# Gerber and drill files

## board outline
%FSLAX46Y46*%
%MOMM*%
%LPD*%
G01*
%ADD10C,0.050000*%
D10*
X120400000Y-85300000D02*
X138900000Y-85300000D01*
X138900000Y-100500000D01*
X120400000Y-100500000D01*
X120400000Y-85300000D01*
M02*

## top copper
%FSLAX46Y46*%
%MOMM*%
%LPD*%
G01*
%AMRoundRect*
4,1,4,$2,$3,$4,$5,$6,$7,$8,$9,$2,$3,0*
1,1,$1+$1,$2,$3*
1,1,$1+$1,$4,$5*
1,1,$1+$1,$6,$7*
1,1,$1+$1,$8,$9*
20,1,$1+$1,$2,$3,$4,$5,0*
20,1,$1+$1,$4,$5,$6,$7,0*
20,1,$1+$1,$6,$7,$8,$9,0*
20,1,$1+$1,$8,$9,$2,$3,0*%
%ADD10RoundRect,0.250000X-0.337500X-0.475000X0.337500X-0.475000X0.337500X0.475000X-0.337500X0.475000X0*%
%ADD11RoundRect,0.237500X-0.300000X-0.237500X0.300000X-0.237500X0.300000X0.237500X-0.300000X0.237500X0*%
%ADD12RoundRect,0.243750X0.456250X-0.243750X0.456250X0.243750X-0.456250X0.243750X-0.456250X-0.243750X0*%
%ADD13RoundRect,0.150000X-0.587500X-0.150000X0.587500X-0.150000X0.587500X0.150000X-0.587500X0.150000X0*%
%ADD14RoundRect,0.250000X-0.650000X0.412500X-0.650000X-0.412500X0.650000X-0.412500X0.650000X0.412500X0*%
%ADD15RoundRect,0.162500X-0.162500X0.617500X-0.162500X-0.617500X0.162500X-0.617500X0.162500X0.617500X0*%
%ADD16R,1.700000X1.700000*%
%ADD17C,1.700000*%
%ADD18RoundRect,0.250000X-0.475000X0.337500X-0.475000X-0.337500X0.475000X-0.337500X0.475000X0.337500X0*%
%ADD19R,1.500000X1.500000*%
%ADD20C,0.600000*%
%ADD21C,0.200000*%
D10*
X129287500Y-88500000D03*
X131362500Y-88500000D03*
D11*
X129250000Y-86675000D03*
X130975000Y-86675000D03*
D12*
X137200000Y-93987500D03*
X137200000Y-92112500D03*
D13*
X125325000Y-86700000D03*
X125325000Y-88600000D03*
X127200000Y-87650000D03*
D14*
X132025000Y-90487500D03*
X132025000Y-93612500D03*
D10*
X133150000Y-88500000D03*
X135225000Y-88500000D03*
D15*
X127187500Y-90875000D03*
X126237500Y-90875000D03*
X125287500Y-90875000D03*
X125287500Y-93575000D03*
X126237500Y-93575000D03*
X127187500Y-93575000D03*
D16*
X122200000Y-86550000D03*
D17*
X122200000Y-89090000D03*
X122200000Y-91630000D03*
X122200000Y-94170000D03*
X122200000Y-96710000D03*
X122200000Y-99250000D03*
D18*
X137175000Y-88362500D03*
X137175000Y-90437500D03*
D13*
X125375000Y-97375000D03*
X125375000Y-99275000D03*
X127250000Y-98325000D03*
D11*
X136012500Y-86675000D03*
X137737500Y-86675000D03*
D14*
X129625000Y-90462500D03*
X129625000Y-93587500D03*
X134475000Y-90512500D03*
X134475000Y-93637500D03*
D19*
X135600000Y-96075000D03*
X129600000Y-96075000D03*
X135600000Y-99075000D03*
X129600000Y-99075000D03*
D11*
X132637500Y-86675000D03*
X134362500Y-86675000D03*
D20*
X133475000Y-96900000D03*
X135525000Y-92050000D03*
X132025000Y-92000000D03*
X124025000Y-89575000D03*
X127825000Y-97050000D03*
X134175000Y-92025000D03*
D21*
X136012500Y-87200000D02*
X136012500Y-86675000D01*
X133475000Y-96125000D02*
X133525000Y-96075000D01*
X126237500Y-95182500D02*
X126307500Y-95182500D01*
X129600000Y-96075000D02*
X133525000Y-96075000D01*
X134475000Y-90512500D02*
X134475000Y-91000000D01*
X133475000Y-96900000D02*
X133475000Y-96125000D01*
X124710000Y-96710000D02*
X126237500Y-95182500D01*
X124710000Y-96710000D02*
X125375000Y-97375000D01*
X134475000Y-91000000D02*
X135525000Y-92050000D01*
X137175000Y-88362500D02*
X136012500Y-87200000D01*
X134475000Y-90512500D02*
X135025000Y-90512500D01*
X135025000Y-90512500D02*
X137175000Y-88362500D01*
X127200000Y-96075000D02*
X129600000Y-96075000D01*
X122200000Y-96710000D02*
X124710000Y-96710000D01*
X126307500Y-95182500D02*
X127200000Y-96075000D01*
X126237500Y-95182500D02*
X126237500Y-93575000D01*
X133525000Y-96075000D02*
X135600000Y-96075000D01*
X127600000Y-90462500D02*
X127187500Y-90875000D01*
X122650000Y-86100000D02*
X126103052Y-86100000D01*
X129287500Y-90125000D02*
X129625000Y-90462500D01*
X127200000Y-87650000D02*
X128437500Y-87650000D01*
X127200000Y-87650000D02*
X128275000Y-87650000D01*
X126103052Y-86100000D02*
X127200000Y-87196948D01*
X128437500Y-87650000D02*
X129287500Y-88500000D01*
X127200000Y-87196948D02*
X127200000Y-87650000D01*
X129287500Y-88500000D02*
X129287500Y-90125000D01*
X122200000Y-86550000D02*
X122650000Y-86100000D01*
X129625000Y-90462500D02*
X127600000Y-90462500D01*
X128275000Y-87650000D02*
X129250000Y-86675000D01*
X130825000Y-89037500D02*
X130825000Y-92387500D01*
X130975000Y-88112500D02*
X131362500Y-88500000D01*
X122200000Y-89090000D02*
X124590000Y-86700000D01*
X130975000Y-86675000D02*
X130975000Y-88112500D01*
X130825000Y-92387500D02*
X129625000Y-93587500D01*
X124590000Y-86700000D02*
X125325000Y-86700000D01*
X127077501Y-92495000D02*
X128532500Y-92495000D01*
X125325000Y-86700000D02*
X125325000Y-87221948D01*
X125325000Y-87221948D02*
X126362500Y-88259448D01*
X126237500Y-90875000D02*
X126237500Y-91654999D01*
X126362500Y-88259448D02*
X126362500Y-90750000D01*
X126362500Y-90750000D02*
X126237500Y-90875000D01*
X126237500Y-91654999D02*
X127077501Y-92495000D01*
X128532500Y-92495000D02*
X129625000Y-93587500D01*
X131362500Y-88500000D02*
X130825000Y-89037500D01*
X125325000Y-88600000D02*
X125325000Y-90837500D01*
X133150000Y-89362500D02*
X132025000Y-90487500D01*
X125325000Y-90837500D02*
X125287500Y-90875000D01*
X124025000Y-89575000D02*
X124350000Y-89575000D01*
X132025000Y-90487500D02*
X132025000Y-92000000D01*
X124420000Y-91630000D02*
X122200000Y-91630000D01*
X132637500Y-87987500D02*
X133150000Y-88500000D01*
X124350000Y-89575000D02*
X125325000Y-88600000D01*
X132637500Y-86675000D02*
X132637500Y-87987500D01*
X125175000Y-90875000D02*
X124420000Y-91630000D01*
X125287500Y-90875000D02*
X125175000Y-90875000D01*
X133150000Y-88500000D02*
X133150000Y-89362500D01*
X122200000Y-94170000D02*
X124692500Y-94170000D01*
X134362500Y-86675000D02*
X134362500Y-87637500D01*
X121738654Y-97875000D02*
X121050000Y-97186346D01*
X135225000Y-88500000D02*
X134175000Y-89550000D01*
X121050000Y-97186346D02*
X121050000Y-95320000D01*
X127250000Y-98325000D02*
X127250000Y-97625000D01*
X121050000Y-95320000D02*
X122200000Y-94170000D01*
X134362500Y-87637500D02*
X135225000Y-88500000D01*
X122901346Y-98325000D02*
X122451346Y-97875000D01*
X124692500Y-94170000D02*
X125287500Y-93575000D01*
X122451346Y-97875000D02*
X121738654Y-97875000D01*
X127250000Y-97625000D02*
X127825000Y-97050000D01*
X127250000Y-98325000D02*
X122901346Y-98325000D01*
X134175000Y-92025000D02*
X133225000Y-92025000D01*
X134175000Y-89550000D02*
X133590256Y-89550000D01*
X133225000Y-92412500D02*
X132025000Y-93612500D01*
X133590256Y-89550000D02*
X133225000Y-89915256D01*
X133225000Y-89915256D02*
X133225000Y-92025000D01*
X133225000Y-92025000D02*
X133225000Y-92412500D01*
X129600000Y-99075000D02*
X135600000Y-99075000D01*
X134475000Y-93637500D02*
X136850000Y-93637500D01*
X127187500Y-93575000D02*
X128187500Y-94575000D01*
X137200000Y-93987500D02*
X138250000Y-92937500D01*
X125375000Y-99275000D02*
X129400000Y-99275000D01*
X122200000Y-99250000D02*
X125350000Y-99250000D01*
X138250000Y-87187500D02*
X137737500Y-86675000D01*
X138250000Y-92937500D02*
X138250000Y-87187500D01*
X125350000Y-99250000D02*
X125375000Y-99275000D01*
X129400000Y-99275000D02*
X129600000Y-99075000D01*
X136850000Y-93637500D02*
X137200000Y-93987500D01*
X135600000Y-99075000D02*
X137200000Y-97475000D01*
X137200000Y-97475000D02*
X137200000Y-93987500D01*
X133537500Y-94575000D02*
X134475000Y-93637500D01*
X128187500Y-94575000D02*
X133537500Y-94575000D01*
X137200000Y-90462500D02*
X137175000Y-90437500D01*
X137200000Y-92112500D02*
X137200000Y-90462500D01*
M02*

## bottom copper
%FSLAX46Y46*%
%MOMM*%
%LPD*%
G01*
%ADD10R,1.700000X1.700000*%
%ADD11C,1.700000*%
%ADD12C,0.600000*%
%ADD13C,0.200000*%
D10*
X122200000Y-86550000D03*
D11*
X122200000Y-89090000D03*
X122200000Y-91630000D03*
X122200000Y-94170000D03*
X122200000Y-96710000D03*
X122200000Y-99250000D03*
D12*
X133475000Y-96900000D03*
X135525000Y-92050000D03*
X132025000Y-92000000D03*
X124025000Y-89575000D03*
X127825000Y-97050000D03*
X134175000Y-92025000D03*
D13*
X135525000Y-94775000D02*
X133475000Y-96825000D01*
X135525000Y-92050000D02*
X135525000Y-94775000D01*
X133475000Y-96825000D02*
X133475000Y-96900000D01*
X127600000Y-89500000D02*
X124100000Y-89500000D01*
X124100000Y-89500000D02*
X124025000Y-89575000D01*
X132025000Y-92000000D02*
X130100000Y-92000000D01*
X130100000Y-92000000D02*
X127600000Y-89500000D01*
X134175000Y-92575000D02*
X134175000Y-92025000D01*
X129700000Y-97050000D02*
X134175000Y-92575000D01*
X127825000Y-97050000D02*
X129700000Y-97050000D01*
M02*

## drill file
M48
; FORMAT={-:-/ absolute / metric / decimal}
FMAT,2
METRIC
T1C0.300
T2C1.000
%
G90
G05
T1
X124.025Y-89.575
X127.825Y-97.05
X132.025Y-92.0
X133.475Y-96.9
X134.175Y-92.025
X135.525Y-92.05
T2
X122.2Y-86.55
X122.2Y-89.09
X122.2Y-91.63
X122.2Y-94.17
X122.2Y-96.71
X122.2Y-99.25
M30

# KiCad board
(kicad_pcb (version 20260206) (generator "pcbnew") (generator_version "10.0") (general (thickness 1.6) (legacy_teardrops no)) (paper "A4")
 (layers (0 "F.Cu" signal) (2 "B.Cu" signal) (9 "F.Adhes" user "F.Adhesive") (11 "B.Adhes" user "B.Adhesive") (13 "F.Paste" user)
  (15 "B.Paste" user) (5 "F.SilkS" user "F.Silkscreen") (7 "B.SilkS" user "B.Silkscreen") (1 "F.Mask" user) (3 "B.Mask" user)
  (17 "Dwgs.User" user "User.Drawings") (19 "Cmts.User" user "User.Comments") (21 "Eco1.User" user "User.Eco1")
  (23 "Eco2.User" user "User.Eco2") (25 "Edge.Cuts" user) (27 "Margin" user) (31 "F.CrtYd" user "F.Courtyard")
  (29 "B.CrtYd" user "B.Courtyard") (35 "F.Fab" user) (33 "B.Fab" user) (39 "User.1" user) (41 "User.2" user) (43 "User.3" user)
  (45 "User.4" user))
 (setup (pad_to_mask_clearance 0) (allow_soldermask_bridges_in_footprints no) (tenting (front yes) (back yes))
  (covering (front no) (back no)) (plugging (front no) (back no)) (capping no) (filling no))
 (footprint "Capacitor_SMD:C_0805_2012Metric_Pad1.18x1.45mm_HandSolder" (layer "F.Cu") (at 130.325 88.5)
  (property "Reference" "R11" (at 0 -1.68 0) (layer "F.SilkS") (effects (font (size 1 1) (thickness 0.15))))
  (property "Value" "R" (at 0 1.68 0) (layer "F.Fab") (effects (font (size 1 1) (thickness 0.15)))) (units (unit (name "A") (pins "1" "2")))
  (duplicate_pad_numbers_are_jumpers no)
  (pad "1" smd roundrect (at -1.0375 0) (size 1.175 1.45) (layers "F.Cu" "F.Mask" "F.Paste") (roundrect_rratio 0.212766)
   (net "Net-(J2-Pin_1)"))
  (pad "2" smd roundrect (at 1.0375 0) (size 1.175 1.45) (layers "F.Cu" "F.Mask" "F.Paste") (roundrect_rratio 0.212766)
   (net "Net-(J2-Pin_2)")))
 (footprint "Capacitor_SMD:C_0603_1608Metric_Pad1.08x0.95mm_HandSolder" (layer "F.Cu") (at 130.1125 86.675)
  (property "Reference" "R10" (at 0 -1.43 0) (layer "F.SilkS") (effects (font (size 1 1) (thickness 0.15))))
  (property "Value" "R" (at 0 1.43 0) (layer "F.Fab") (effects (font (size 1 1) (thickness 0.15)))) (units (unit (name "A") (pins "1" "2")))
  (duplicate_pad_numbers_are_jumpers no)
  (pad "1" smd roundrect (at -0.8625 0) (size 1.075 0.95) (layers "F.Cu" "F.Mask" "F.Paste") (roundrect_rratio 0.25) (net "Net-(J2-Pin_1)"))
  (pad "2" smd roundrect (at 0.8625 0) (size 1.075 0.95) (layers "F.Cu" "F.Mask" "F.Paste") (roundrect_rratio 0.25) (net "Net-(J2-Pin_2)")))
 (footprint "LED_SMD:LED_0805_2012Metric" (layer "F.Cu") (at 137.2 93.05 90)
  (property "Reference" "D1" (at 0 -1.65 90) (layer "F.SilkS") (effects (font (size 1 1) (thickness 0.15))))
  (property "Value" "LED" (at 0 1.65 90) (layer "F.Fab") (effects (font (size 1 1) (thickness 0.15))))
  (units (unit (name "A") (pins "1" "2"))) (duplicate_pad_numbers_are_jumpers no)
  (pad "1" smd roundrect (at -0.9375 0 90) (size 0.975 1.4) (layers "F.Cu" "F.Mask" "F.Paste") (roundrect_rratio 0.25) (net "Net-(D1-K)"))
  (pad "2" smd roundrect (at 0.9375 0 90) (size 0.975 1.4) (layers "F.Cu" "F.Mask" "F.Paste") (roundrect_rratio 0.25) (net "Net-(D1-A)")))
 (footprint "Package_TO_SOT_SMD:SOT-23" (layer "F.Cu") (at 126.2625 87.65)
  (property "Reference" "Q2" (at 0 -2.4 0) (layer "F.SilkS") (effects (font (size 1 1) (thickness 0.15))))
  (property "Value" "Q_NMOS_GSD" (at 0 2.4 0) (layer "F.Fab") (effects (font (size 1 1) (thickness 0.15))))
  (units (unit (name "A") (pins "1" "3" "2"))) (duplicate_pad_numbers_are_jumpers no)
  (pad "1" smd roundrect (at -0.9375 -0.95) (size 1.475 0.6) (layers "F.Cu" "F.Mask" "F.Paste") (roundrect_rratio 0.25)
   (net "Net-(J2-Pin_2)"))
  (pad "2" smd roundrect (at -0.9375 0.95) (size 1.475 0.6) (layers "F.Cu" "F.Mask" "F.Paste") (roundrect_rratio 0.25)
   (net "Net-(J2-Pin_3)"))
  (pad "3" smd roundrect (at 0.9375 0) (size 1.475 0.6) (layers "F.Cu" "F.Mask" "F.Paste") (roundrect_rratio 0.25) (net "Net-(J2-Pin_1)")))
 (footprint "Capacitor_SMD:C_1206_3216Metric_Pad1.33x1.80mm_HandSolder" (layer "F.Cu") (at 132.025 92.05 -90)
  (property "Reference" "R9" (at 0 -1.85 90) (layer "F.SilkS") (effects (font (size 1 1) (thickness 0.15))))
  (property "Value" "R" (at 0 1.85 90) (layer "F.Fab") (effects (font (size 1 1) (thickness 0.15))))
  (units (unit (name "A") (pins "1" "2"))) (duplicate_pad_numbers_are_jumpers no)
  (pad "1" smd roundrect (at -1.5625 0 270) (size 1.325 1.8) (layers "F.Cu" "F.Mask" "F.Paste") (roundrect_rratio 0.188679)
   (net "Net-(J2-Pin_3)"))
  (pad "2" smd roundrect (at 1.5625 0 270) (size 1.325 1.8) (layers "F.Cu" "F.Mask" "F.Paste") (roundrect_rratio 0.188679)
   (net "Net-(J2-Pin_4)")))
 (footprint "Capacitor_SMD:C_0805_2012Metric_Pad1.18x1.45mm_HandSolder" (layer "F.Cu") (at 134.1875 88.5)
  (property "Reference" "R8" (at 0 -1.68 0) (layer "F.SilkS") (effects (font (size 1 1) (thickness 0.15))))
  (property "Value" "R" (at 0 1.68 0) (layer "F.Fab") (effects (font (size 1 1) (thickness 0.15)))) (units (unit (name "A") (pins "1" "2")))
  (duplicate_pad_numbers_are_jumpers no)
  (pad "1" smd roundrect (at -1.0375 0) (size 1.175 1.45) (layers "F.Cu" "F.Mask" "F.Paste") (roundrect_rratio 0.212766)
   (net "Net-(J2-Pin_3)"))
  (pad "2" smd roundrect (at 1.0375 0) (size 1.175 1.45) (layers "F.Cu" "F.Mask" "F.Paste") (roundrect_rratio 0.212766)
   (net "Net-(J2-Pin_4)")))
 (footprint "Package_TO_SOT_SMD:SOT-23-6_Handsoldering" (layer "F.Cu") (at 126.2375 92.225 -90)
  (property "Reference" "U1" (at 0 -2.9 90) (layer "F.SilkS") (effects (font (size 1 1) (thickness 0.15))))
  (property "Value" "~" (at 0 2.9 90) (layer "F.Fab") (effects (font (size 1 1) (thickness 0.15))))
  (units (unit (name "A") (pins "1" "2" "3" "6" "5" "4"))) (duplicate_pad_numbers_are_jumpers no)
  (pad "1" smd roundrect (at -1.35 -0.95 270) (size 1.56 0.65) (layers "F.Cu" "F.Mask" "F.Paste") (roundrect_rratio 0.25)
   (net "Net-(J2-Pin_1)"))
  (pad "2" smd roundrect (at -1.35 0 270) (size 1.56 0.65) (layers "F.Cu" "F.Mask" "F.Paste") (roundrect_rratio 0.25) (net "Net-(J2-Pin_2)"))
  (pad "3" smd roundrect (at -1.35 0.95 270) (size 1.56 0.65) (layers "F.Cu" "F.Mask" "F.Paste") (roundrect_rratio 0.25)
   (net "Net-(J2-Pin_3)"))
  (pad "4" smd roundrect (at 1.35 0.95 270) (size 1.56 0.65) (layers "F.Cu" "F.Mask" "F.Paste") (roundrect_rratio 0.25)
   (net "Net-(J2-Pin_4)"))
  (pad "5" smd roundrect (at 1.35 0 270) (size 1.56 0.65) (layers "F.Cu" "F.Mask" "F.Paste") (roundrect_rratio 0.25) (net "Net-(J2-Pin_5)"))
  (pad "6" smd roundrect (at 1.35 -0.95 270) (size 1.56 0.65) (layers "F.Cu" "F.Mask" "F.Paste") (roundrect_rratio 0.25) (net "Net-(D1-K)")))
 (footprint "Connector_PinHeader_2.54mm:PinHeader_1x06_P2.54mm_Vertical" (layer "F.Cu") (at 122.2 86.55)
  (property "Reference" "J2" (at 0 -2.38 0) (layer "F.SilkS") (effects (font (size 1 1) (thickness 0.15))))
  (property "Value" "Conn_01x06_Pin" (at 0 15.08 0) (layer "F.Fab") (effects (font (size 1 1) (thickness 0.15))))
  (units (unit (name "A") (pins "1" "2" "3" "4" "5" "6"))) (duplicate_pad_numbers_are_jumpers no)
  (pad "1" thru_hole rect (at 0 0) (size 1.7 1.7) (drill 1) (layers "*.Cu" "*.Mask") (remove_unused_layers no) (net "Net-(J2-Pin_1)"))
  (pad "2" thru_hole circle (at 0 2.54) (size 1.7 1.7) (drill 1) (layers "*.Cu" "*.Mask") (remove_unused_layers no) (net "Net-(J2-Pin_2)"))
  (pad "3" thru_hole circle (at 0 5.08) (size 1.7 1.7) (drill 1) (layers "*.Cu" "*.Mask") (remove_unused_layers no) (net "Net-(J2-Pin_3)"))
  (pad "4" thru_hole circle (at 0 7.62) (size 1.7 1.7) (drill 1) (layers "*.Cu" "*.Mask") (remove_unused_layers no) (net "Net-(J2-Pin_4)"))
  (pad "5" thru_hole circle (at 0 10.16) (size 1.7 1.7) (drill 1) (layers "*.Cu" "*.Mask") (remove_unused_layers no) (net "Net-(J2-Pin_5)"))
  (pad "6" thru_hole circle (at 0 12.7) (size 1.7 1.7) (drill 1) (layers "*.Cu" "*.Mask") (remove_unused_layers no) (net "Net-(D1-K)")))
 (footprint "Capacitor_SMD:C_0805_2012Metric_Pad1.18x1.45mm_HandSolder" (layer "F.Cu") (at 137.175 89.4 -90)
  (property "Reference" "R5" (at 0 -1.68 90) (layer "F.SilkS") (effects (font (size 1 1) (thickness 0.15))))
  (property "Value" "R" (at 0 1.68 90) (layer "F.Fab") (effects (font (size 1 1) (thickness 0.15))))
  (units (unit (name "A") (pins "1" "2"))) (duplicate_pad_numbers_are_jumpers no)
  (pad "1" smd roundrect (at -1.0375 0 270) (size 1.175 1.45) (layers "F.Cu" "F.Mask" "F.Paste") (roundrect_rratio 0.212766)
   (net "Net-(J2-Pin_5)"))
  (pad "2" smd roundrect (at 1.0375 0 270) (size 1.175 1.45) (layers "F.Cu" "F.Mask" "F.Paste") (roundrect_rratio 0.212766)
   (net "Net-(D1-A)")))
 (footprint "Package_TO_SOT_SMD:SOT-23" (layer "F.Cu") (at 126.3125 98.325)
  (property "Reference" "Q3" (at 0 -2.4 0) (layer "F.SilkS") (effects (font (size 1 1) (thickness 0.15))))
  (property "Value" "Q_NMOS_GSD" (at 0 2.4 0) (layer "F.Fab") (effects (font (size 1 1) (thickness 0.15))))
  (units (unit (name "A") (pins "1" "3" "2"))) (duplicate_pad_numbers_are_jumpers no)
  (pad "1" smd roundrect (at -0.9375 -0.95) (size 1.475 0.6) (layers "F.Cu" "F.Mask" "F.Paste") (roundrect_rratio 0.25)
   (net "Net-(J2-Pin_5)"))
  (pad "2" smd roundrect (at -0.9375 0.95) (size 1.475 0.6) (layers "F.Cu" "F.Mask" "F.Paste") (roundrect_rratio 0.25) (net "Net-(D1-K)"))
  (pad "3" smd roundrect (at 0.9375 0) (size 1.475 0.6) (layers "F.Cu" "F.Mask" "F.Paste") (roundrect_rratio 0.25) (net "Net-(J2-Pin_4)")))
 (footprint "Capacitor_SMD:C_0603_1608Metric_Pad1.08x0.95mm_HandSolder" (layer "F.Cu") (at 136.875 86.675)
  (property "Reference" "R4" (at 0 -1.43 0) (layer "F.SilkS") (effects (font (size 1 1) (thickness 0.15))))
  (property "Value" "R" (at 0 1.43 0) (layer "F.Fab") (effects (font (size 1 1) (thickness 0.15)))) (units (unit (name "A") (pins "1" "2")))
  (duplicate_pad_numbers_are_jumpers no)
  (pad "1" smd roundrect (at -0.8625 0) (size 1.075 0.95) (layers "F.Cu" "F.Mask" "F.Paste") (roundrect_rratio 0.25) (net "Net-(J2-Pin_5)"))
  (pad "2" smd roundrect (at 0.8625 0) (size 1.075 0.95) (layers "F.Cu" "F.Mask" "F.Paste") (roundrect_rratio 0.25) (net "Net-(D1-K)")))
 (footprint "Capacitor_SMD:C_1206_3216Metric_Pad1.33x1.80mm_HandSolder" (layer "F.Cu") (at 129.625 92.025 -90)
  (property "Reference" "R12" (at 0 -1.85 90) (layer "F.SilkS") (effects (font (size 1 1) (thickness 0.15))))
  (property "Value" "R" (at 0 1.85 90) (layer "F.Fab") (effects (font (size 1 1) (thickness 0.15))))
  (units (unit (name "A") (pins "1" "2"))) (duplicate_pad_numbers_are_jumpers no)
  (pad "1" smd roundrect (at -1.5625 0 270) (size 1.325 1.8) (layers "F.Cu" "F.Mask" "F.Paste") (roundrect_rratio 0.188679)
   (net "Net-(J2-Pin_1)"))
  (pad "2" smd roundrect (at 1.5625 0 270) (size 1.325 1.8) (layers "F.Cu" "F.Mask" "F.Paste") (roundrect_rratio 0.188679)
   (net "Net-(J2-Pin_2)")))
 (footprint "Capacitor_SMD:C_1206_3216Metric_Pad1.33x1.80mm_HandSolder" (layer "F.Cu") (at 134.475 92.075 -90)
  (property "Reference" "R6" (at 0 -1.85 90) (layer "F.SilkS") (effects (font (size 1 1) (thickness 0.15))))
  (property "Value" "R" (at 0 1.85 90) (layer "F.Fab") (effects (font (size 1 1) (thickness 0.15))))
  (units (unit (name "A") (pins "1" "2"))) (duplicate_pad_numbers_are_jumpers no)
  (pad "1" smd roundrect (at -1.5625 0 270) (size 1.325 1.8) (layers "F.Cu" "F.Mask" "F.Paste") (roundrect_rratio 0.188679)
   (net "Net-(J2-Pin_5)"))
  (pad "2" smd roundrect (at 1.5625 0 270) (size 1.325 1.8) (layers "F.Cu" "F.Mask" "F.Paste") (roundrect_rratio 0.188679)
   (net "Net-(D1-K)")))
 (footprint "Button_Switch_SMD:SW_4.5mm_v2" (layer "F.Cu") (at 132.6 97.575 -90)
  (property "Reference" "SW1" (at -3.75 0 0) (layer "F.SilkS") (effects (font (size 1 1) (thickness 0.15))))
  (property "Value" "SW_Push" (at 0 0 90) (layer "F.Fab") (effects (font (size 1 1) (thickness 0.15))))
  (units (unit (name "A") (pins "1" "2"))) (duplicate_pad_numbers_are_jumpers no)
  (pad "1" smd rect (at -1.5 -3 270) (size 1.5 1.5) (layers "F.Cu" "F.Mask" "F.Paste") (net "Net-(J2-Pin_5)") (thermal_bridge_angle 45))
  (pad "1" smd rect (at -1.5 3 270) (size 1.5 1.5) (layers "F.Cu" "F.Mask" "F.Paste") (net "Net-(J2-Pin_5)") (thermal_bridge_angle 45))
  (pad "2" smd rect (at 1.5 -3 270) (size 1.5 1.5) (layers "F.Cu" "F.Mask" "F.Paste") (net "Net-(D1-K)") (thermal_bridge_angle 45))
  (pad "2" smd rect (at 1.5 3 270) (size 1.5 1.5) (layers "F.Cu" "F.Mask" "F.Paste") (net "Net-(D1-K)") (thermal_bridge_angle 45)))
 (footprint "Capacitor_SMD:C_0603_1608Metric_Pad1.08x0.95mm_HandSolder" (layer "F.Cu") (at 133.5 86.675)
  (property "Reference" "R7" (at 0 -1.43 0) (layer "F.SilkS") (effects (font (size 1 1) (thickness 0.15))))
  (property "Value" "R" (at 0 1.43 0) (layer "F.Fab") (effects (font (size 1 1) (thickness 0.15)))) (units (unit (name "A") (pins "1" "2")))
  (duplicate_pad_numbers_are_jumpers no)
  (pad "1" smd roundrect (at -0.8625 0) (size 1.075 0.95) (layers "F.Cu" "F.Mask" "F.Paste") (roundrect_rratio 0.25) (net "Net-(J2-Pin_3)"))
  (pad "2" smd roundrect (at 0.8625 0) (size 1.075 0.95) (layers "F.Cu" "F.Mask" "F.Paste") (roundrect_rratio 0.25) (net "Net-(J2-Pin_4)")))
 (gr_rect (start 120.4 85.3) (end 138.9 100.5) (stroke (width 0.05) (type default)) (fill no) (layer "Edge.Cuts"))
 (segment (start 136.0125 87.2) (end 136.0125 86.675) (width 0.2) (layer "F.Cu") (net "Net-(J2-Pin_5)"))
 (segment (start 133.475 96.125) (end 133.525 96.075) (width 0.2) (layer "F.Cu") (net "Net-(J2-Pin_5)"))
 (segment (start 126.2375 95.1825) (end 126.3075 95.1825) (width 0.2) (layer "F.Cu") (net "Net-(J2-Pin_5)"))
 (segment (start 129.6 96.075) (end 133.525 96.075) (width 0.2) (layer "F.Cu") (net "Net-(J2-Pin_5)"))
 (segment (start 134.475 90.5125) (end 134.475 91) (width 0.2) (layer "F.Cu") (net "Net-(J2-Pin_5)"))
 (segment (start 133.475 96.9) (end 133.475 96.125) (width 0.2) (layer "F.Cu") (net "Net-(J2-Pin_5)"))
 (segment (start 124.71 96.71) (end 126.2375 95.1825) (width 0.2) (layer "F.Cu") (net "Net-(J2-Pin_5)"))
 (segment (start 124.71 96.71) (end 125.375 97.375) (width 0.2) (layer "F.Cu") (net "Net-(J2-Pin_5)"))
 (segment (start 134.475 91) (end 135.525 92.05) (width 0.2) (layer "F.Cu") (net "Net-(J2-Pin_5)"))
 (segment (start 137.175 88.3625) (end 136.0125 87.2) (width 0.2) (layer "F.Cu") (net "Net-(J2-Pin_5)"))
 (segment (start 134.475 90.5125) (end 135.025 90.5125) (width 0.2) (layer "F.Cu") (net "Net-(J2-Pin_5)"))
 (segment (start 135.025 90.5125) (end 137.175 88.3625) (width 0.2) (layer "F.Cu") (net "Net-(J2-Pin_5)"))
 (segment (start 127.2 96.075) (end 129.6 96.075) (width 0.2) (layer "F.Cu") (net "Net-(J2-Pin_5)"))
 (segment (start 122.2 96.71) (end 124.71 96.71) (width 0.2) (layer "F.Cu") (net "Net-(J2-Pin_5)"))
 (segment (start 126.3075 95.1825) (end 127.2 96.075) (width 0.2) (layer "F.Cu") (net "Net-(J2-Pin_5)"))
 (segment (start 126.2375 95.1825) (end 126.2375 93.575) (width 0.2) (layer "F.Cu") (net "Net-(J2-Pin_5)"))
 (segment (start 133.525 96.075) (end 135.6 96.075) (width 0.2) (layer "F.Cu") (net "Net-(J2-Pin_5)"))
 (via (at 133.475 96.9) (size 0.6) (drill 0.3) (layers "F.Cu" "B.Cu") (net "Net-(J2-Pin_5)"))
 (via (at 135.525 92.05) (size 0.6) (drill 0.3) (layers "F.Cu" "B.Cu") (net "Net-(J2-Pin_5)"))
 (segment (start 135.525 94.775) (end 133.475 96.825) (width 0.2) (layer "B.Cu") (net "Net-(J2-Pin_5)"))
 (segment (start 135.525 92.05) (end 135.525 94.775) (width 0.2) (layer "B.Cu") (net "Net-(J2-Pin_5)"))
 (segment (start 133.475 96.825) (end 133.475 96.9) (width 0.2) (layer "B.Cu") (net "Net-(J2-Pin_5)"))
 (segment (start 127.6 90.4625) (end 127.1875 90.875) (width 0.2) (layer "F.Cu") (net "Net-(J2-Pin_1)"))
 (segment (start 122.65 86.1) (end 126.103052 86.1) (width 0.2) (layer "F.Cu") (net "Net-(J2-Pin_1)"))
 (segment (start 129.2875 90.125) (end 129.625 90.4625) (width 0.2) (layer "F.Cu") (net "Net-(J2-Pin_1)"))
 (segment (start 127.2 87.65) (end 128.4375 87.65) (width 0.2) (layer "F.Cu") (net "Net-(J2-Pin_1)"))
 (segment (start 127.2 87.65) (end 128.275 87.65) (width 0.2) (layer "F.Cu") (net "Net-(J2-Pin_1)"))
 (segment (start 126.103052 86.1) (end 127.2 87.196948) (width 0.2) (layer "F.Cu") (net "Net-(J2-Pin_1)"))
 (segment (start 128.4375 87.65) (end 129.2875 88.5) (width 0.2) (layer "F.Cu") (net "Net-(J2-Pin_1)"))
 (segment (start 127.2 87.196948) (end 127.2 87.65) (width 0.2) (layer "F.Cu") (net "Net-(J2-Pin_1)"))
 (segment (start 129.2875 88.5) (end 129.2875 90.125) (width 0.2) (layer "F.Cu") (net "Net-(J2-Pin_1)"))
 (segment (start 122.2 86.55) (end 122.65 86.1) (width 0.2) (layer "F.Cu") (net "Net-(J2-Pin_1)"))
 (segment (start 129.625 90.4625) (end 127.6 90.4625) (width 0.2) (layer "F.Cu") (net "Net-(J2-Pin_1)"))
 (segment (start 128.275 87.65) (end 129.25 86.675) (width 0.2) (layer "F.Cu") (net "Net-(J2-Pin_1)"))
 (segment (start 130.825 89.0375) (end 130.825 92.3875) (width 0.2) (layer "F.Cu") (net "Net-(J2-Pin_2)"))
 (segment (start 130.975 88.1125) (end 131.3625 88.5) (width 0.2) (layer "F.Cu") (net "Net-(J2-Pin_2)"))
 (segment (start 122.2 89.09) (end 124.59 86.7) (width 0.2) (layer "F.Cu") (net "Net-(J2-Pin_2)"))
 (segment (start 130.975 86.675) (end 130.975 88.1125) (width 0.2) (layer "F.Cu") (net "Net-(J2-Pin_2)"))
 (segment (start 130.825 92.3875) (end 129.625 93.5875) (width 0.2) (layer "F.Cu") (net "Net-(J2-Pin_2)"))
 (segment (start 124.59 86.7) (end 125.325 86.7) (width 0.2) (layer "F.Cu") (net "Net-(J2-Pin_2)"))
 (segment (start 127.077501 92.495) (end 128.5325 92.495) (width 0.2) (layer "F.Cu") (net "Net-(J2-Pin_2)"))
 (segment (start 125.325 86.7) (end 125.325 87.221948) (width 0.2) (layer "F.Cu") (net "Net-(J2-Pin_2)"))
 (segment (start 125.325 87.221948) (end 126.3625 88.259448) (width 0.2) (layer "F.Cu") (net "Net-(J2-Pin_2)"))
 (segment (start 126.2375 90.875) (end 126.2375 91.654999) (width 0.2) (layer "F.Cu") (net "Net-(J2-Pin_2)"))
 (segment (start 126.3625 88.259448) (end 126.3625 90.75) (width 0.2) (layer "F.Cu") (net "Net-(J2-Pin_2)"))
 (segment (start 126.3625 90.75) (end 126.2375 90.875) (width 0.2) (layer "F.Cu") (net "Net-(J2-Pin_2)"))
 (segment (start 126.2375 91.654999) (end 127.077501 92.495) (width 0.2) (layer "F.Cu") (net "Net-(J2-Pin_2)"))
 (segment (start 128.5325 92.495) (end 129.625 93.5875) (width 0.2) (layer "F.Cu") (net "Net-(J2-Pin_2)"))
 (segment (start 131.3625 88.5) (end 130.825 89.0375) (width 0.2) (layer "F.Cu") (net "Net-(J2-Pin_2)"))
 (segment (start 125.325 88.6) (end 125.325 90.8375) (width 0.2) (layer "F.Cu") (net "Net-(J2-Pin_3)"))
 (segment (start 133.15 89.3625) (end 132.025 90.4875) (width 0.2) (layer "F.Cu") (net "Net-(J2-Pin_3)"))
 (segment (start 125.325 90.8375) (end 125.2875 90.875) (width 0.2) (layer "F.Cu") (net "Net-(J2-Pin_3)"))
 (segment (start 124.025 89.575) (end 124.35 89.575) (width 0.2) (layer "F.Cu") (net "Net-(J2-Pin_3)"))
 (segment (start 132.025 90.4875) (end 132.025 92) (width 0.2) (layer "F.Cu") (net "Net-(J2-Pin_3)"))
 (segment (start 124.42 91.63) (end 122.2 91.63) (width 0.2) (layer "F.Cu") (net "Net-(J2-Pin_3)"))
 (segment (start 132.6375 87.9875) (end 133.15 88.5) (width 0.2) (layer "F.Cu") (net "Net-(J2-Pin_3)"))
 (segment (start 124.35 89.575) (end 125.325 88.6) (width 0.2) (layer "F.Cu") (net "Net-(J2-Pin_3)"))
 (segment (start 132.6375 86.675) (end 132.6375 87.9875) (width 0.2) (layer "F.Cu") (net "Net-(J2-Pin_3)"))
 (segment (start 125.175 90.875) (end 124.42 91.63) (width 0.2) (layer "F.Cu") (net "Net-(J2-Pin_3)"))
 (segment (start 125.2875 90.875) (end 125.175 90.875) (width 0.2) (layer "F.Cu") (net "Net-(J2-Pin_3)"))
 (segment (start 133.15 88.5) (end 133.15 89.3625) (width 0.2) (layer "F.Cu") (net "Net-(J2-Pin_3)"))
 (via (at 132.025 92) (size 0.6) (drill 0.3) (layers "F.Cu" "B.Cu") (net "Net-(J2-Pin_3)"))
 (via (at 124.025 89.575) (size 0.6) (drill 0.3) (layers "F.Cu" "B.Cu") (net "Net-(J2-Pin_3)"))
 (segment (start 127.6 89.5) (end 124.1 89.5) (width 0.2) (layer "B.Cu") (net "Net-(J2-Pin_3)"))
 (segment (start 124.1 89.5) (end 124.025 89.575) (width 0.2) (layer "B.Cu") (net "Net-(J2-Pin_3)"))
 (segment (start 132.025 92) (end 130.1 92) (width 0.2) (layer "B.Cu") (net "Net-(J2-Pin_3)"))
 (segment (start 130.1 92) (end 127.6 89.5) (width 0.2) (layer "B.Cu") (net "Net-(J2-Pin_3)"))
 (segment (start 122.2 94.17) (end 124.6925 94.17) (width 0.2) (layer "F.Cu") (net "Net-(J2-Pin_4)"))
 (segment (start 134.3625 86.675) (end 134.3625 87.6375) (width 0.2) (layer "F.Cu") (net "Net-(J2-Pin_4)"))
 (segment (start 121.738654 97.875) (end 121.05 97.186346) (width 0.2) (layer "F.Cu") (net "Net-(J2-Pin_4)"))
 (segment (start 135.225 88.5) (end 134.175 89.55) (width 0.2) (layer "F.Cu") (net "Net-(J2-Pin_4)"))
 (segment (start 121.05 97.186346) (end 121.05 95.32) (width 0.2) (layer "F.Cu") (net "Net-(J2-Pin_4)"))
 (segment (start 127.25 98.325) (end 127.25 97.625) (width 0.2) (layer "F.Cu") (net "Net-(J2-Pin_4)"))
 (segment (start 121.05 95.32) (end 122.2 94.17) (width 0.2) (layer "F.Cu") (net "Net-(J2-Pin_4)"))
 (segment (start 134.3625 87.6375) (end 135.225 88.5) (width 0.2) (layer "F.Cu") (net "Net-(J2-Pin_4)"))
 (segment (start 122.901346 98.325) (end 122.451346 97.875) (width 0.2) (layer "F.Cu") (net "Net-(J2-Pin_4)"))
 (segment (start 124.6925 94.17) (end 125.2875 93.575) (width 0.2) (layer "F.Cu") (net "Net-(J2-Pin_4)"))
 (segment (start 122.451346 97.875) (end 121.738654 97.875) (width 0.2) (layer "F.Cu") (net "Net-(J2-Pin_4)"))
 (segment (start 127.25 97.625) (end 127.825 97.05) (width 0.2) (layer "F.Cu") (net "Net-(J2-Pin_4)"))
 (segment (start 127.25 98.325) (end 122.901346 98.325) (width 0.2) (layer "F.Cu") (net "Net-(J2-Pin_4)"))
 (segment (start 134.175 92.025) (end 133.225 92.025) (width 0.2) (layer "F.Cu") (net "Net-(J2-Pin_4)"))
 (segment (start 134.175 89.55) (end 133.590256 89.55) (width 0.2) (layer "F.Cu") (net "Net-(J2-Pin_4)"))
 (segment (start 133.225 92.4125) (end 132.025 93.6125) (width 0.2) (layer "F.Cu") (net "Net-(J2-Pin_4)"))
 (segment (start 133.590256 89.55) (end 133.225 89.915256) (width 0.2) (layer "F.Cu") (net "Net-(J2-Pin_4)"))
 (segment (start 133.225 89.915256) (end 133.225 92.025) (width 0.2) (layer "F.Cu") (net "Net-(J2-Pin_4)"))
 (segment (start 133.225 92.025) (end 133.225 92.4125) (width 0.2) (layer "F.Cu") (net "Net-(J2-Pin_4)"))
 (via (at 127.825 97.05) (size 0.6) (drill 0.3) (layers "F.Cu" "B.Cu") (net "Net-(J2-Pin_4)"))
 (via (at 134.175 92.025) (size 0.6) (drill 0.3) (layers "F.Cu" "B.Cu") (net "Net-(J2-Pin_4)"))
 (segment (start 134.175 92.575) (end 134.175 92.025) (width 0.2) (layer "B.Cu") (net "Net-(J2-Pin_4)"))
 (segment (start 129.7 97.05) (end 134.175 92.575) (width 0.2) (layer "B.Cu") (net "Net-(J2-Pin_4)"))
 (segment (start 127.825 97.05) (end 129.7 97.05) (width 0.2) (layer "B.Cu") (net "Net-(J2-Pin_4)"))
 (segment (start 129.6 99.075) (end 135.6 99.075) (width 0.2) (layer "F.Cu") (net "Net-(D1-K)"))
 (segment (start 134.475 93.6375) (end 136.85 93.6375) (width 0.2) (layer "F.Cu") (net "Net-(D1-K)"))
 (segment (start 127.1875 93.575) (end 128.1875 94.575) (width 0.2) (layer "F.Cu") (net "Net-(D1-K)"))
 (segment (start 137.2 93.9875) (end 138.25 92.9375) (width 0.2) (layer "F.Cu") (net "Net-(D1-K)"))
 (segment (start 125.375 99.275) (end 129.4 99.275) (width 0.2) (layer "F.Cu") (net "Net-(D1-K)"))
 (segment (start 122.2 99.25) (end 125.35 99.25) (width 0.2) (layer "F.Cu") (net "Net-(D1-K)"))
 (segment (start 138.25 87.1875) (end 137.7375 86.675) (width 0.2) (layer "F.Cu") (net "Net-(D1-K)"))
 (segment (start 138.25 92.9375) (end 138.25 87.1875) (width 0.2) (layer "F.Cu") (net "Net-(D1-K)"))
 (segment (start 125.35 99.25) (end 125.375 99.275) (width 0.2) (layer "F.Cu") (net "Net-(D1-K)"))
 (segment (start 129.4 99.275) (end 129.6 99.075) (width 0.2) (layer "F.Cu") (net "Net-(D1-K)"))
 (segment (start 136.85 93.6375) (end 137.2 93.9875) (width 0.2) (layer "F.Cu") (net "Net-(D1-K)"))
 (segment (start 135.6 99.075) (end 137.2 97.475) (width 0.2) (layer "F.Cu") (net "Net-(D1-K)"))
 (segment (start 137.2 97.475) (end 137.2 93.9875) (width 0.2) (layer "F.Cu") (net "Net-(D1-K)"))
 (segment (start 133.5375 94.575) (end 134.475 93.6375) (width 0.2) (layer "F.Cu") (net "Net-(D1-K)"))
 (segment (start 128.1875 94.575) (end 133.5375 94.575) (width 0.2) (layer "F.Cu") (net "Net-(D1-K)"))
 (segment (start 137.2 90.4625) (end 137.175 90.4375) (width 0.2) (layer "F.Cu") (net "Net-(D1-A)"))
 (segment (start 137.2 92.1125) (end 137.2 90.4625) (width 0.2) (layer "F.Cu") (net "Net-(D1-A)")))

